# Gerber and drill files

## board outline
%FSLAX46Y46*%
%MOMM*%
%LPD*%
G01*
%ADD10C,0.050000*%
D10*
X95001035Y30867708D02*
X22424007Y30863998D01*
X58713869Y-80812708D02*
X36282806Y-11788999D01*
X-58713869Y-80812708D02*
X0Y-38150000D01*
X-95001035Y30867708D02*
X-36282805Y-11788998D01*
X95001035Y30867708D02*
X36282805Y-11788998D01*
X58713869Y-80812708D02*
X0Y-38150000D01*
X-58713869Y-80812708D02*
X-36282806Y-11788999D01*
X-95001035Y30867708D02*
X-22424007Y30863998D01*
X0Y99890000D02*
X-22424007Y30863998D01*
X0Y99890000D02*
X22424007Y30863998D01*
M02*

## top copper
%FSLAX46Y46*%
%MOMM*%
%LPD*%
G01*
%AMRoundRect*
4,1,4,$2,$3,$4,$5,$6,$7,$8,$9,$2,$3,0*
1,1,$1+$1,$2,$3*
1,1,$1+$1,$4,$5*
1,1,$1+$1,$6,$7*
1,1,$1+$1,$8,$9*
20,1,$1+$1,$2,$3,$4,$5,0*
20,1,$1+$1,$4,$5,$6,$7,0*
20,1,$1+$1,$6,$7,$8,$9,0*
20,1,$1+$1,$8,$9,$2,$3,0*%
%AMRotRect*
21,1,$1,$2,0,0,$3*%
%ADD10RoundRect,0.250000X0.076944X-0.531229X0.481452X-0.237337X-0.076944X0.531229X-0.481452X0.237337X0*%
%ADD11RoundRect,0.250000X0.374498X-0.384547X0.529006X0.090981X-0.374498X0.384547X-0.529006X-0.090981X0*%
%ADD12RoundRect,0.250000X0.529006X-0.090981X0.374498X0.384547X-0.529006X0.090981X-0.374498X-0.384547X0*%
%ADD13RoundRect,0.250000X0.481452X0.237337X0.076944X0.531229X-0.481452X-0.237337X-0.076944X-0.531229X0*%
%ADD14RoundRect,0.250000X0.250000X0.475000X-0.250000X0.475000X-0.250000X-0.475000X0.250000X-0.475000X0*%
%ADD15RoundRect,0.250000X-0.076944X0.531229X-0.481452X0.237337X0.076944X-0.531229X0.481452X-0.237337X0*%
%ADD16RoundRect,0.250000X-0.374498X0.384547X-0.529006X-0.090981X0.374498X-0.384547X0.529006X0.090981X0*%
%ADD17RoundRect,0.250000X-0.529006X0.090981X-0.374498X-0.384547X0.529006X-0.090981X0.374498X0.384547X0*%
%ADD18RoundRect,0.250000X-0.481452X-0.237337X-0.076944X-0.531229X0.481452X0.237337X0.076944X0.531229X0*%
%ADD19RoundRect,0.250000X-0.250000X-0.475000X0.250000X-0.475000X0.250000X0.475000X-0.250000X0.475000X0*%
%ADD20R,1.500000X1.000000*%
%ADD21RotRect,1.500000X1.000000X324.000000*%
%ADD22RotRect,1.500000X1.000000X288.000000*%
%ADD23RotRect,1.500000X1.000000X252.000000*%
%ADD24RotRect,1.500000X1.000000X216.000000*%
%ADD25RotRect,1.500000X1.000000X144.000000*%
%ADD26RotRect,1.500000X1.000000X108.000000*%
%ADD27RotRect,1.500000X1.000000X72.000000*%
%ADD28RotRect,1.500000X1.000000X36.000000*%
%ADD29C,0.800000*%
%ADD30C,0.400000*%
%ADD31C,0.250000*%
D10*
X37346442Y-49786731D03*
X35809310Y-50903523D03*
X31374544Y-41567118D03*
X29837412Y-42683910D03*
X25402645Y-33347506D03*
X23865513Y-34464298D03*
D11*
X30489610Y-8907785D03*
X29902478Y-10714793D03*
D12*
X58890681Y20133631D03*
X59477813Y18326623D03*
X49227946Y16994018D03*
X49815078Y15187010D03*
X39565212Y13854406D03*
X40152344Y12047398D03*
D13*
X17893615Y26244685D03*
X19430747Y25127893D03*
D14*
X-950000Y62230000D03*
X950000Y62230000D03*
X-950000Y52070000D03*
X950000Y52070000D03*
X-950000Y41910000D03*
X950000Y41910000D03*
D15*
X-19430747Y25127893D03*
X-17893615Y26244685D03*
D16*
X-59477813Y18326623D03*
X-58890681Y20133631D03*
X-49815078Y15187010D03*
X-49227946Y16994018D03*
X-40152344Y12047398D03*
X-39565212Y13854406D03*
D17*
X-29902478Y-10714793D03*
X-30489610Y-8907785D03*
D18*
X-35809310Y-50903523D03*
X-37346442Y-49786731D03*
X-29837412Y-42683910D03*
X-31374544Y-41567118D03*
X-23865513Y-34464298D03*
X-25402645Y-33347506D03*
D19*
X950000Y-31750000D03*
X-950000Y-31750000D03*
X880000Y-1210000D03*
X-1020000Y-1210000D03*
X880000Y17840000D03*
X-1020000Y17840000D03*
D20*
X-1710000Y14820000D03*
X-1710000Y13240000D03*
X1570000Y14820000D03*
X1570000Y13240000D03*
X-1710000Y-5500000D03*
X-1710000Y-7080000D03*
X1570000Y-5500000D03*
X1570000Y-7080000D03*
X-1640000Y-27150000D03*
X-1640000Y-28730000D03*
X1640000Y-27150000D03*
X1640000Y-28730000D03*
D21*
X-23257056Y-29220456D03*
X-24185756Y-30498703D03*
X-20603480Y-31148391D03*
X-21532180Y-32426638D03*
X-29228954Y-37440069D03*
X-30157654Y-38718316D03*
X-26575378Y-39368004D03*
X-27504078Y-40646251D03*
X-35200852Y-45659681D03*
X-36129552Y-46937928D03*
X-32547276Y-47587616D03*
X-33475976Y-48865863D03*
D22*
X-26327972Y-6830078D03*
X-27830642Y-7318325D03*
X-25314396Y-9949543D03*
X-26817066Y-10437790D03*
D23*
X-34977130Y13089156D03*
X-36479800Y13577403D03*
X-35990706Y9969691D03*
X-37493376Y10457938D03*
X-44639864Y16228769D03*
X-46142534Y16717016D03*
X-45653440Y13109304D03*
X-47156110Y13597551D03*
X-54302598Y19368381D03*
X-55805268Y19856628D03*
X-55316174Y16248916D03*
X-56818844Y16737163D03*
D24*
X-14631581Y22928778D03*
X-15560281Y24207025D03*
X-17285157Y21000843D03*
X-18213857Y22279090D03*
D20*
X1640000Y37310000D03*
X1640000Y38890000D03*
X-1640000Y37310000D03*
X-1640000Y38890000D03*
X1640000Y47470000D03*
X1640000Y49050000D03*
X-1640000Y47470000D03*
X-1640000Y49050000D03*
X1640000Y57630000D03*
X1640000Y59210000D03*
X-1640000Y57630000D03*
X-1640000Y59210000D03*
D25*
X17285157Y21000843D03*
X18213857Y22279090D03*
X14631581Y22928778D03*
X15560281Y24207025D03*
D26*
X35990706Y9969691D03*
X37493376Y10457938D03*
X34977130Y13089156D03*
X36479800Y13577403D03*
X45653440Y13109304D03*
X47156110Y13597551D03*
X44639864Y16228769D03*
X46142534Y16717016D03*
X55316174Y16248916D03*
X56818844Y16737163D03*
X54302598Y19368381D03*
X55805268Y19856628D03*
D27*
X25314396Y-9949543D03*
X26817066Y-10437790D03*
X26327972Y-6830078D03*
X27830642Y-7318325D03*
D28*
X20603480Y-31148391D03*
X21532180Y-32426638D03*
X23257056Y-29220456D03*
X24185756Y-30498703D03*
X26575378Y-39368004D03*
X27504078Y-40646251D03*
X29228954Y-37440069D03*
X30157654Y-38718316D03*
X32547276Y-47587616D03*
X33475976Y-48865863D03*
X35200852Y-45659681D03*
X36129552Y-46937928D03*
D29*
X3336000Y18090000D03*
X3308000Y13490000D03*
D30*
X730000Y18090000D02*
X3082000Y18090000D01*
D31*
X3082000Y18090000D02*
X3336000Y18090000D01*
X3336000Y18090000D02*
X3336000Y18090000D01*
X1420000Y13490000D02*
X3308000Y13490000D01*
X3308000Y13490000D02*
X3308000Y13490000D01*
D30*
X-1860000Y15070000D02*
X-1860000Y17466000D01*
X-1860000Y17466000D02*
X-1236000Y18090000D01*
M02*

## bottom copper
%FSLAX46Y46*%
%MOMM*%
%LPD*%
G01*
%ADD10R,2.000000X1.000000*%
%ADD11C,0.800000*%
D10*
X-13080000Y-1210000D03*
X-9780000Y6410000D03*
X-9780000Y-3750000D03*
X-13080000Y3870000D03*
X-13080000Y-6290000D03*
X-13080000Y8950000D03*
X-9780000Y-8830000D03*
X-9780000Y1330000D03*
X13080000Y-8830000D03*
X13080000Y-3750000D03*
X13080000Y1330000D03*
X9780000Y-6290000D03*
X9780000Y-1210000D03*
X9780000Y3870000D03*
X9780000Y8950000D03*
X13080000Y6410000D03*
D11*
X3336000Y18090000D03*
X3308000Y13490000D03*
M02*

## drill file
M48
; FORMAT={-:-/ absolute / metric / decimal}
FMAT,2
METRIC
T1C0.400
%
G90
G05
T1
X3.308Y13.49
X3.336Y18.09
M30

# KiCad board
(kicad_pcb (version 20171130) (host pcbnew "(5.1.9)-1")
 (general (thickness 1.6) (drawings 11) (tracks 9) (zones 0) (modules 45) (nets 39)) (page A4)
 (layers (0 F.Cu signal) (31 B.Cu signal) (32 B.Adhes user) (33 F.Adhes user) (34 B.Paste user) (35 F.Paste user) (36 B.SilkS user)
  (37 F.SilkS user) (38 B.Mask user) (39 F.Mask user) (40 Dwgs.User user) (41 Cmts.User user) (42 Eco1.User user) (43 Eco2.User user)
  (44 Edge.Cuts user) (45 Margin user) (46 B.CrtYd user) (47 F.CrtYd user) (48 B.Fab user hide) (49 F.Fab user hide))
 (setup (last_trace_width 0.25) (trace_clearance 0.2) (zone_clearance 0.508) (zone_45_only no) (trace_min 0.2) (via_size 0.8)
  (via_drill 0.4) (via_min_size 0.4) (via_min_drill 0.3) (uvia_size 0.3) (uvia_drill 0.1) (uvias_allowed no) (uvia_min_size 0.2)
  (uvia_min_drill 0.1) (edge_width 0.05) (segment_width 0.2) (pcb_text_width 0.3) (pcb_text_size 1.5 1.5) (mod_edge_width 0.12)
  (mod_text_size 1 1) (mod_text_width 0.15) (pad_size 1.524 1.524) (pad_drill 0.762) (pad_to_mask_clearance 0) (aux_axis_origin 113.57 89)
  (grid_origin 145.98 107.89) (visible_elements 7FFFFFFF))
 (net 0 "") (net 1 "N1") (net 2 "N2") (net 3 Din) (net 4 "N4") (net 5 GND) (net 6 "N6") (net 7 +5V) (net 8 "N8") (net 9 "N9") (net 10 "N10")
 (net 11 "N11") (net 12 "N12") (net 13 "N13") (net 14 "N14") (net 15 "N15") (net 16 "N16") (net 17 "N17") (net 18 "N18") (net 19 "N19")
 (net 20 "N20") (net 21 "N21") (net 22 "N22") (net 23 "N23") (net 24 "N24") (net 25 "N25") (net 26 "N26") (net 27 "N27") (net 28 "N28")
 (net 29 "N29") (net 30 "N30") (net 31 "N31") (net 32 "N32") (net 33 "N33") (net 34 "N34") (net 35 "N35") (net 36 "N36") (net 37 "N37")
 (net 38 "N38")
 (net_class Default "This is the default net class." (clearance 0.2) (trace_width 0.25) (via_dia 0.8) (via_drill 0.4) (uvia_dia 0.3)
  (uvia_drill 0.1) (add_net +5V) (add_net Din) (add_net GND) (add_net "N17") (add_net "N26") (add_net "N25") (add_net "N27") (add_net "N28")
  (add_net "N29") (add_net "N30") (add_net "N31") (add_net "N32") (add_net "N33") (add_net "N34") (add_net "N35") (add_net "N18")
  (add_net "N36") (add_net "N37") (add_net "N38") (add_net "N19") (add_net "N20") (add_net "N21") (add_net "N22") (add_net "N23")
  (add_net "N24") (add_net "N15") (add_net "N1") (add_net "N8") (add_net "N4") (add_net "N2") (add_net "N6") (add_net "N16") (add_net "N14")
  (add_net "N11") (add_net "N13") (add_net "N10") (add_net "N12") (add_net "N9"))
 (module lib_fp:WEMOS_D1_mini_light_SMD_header (layer B.Cu) (at 0 -0.06 180)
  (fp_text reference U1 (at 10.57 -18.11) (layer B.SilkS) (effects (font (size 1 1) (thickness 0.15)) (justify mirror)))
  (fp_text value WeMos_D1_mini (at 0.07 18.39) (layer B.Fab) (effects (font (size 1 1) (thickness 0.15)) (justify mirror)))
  (pad 12 smd rect (at 13.08 -1.27 180) (size 2 1) (layers B.Cu B.Paste B.Mask) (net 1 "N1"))
  (pad 15 smd rect (at 9.78 6.35 180) (size 2 1) (layers B.Cu B.Paste B.Mask) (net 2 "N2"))
  (pad 11 smd rect (at 9.78 -3.81 180) (size 2 1) (layers B.Cu B.Paste B.Mask) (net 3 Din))
  (pad 14 smd rect (at 13.08 3.81 180) (size 2 1) (layers B.Cu B.Paste B.Mask) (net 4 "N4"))
  (pad 10 smd rect (at 13.08 -6.35 180) (size 2 1) (layers B.Cu B.Paste B.Mask) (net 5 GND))
  (pad 16 smd rect (at 13.08 8.89 180) (size 2 1) (layers B.Cu B.Paste B.Mask) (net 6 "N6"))
  (pad 9 smd rect (at 9.78 -8.89 180) (size 2 1) (layers B.Cu B.Paste B.Mask) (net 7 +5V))
  (pad 13 smd rect (at 9.78 1.27 180) (size 2 1) (layers B.Cu B.Paste B.Mask) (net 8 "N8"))
  (pad 8 smd rect (at -13.08 -8.89 180) (size 2 1) (layers B.Cu B.Paste B.Mask) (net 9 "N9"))
  (pad 6 smd rect (at -13.08 -3.81 180) (size 2 1) (layers B.Cu B.Paste B.Mask) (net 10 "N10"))
  (pad 4 smd rect (at -13.08 1.27 180) (size 2 1) (layers B.Cu B.Paste B.Mask) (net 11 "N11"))
  (pad 7 smd rect (at -9.78 -6.35 180) (size 2 1) (layers B.Cu B.Paste B.Mask) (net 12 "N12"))
  (pad 5 smd rect (at -9.78 -1.27 180) (size 2 1) (layers B.Cu B.Paste B.Mask) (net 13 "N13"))
  (pad 3 smd rect (at -9.78 3.81 180) (size 2 1) (layers B.Cu B.Paste B.Mask) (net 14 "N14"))
  (pad 1 smd rect (at -9.78 8.89 180) (size 2 1) (layers B.Cu B.Paste B.Mask) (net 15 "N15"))
  (pad 2 smd rect (at -13.08 6.35 180) (size 2 1) (layers B.Cu B.Paste B.Mask) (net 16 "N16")))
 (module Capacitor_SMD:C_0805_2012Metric (layer F.Cu) (at 36.577876 50.345127 36)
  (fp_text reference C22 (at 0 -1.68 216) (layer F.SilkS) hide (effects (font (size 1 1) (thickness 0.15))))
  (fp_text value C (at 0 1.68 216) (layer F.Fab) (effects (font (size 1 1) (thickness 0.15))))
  (pad 2 smd roundrect (at 0.95 0 36) (size 1 1.45) (layers F.Cu F.Paste F.Mask) (roundrect_rratio 0.25) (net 5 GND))
  (pad 1 smd roundrect (at -0.95 0 36) (size 1 1.45) (layers F.Cu F.Paste F.Mask) (roundrect_rratio 0.25) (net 7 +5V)))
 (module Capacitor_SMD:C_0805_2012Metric (layer F.Cu) (at 30.605978 42.125514 36)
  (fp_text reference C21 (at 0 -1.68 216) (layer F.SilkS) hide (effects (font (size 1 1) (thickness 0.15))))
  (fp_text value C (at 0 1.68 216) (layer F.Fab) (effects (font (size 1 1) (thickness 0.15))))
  (pad 2 smd roundrect (at 0.95 0 36) (size 1 1.45) (layers F.Cu F.Paste F.Mask) (roundrect_rratio 0.25) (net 5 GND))
  (pad 1 smd roundrect (at -0.95 0 36) (size 1 1.45) (layers F.Cu F.Paste F.Mask) (roundrect_rratio 0.25) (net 7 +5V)))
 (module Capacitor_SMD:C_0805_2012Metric (layer F.Cu) (at 24.634079 33.905902 36)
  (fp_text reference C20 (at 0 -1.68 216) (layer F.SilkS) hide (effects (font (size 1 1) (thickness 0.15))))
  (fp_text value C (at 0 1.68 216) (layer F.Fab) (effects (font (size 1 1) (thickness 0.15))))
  (pad 2 smd roundrect (at 0.95 0 36) (size 1 1.45) (layers F.Cu F.Paste F.Mask) (roundrect_rratio 0.25) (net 5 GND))
  (pad 1 smd roundrect (at -0.95 0 36) (size 1 1.45) (layers F.Cu F.Paste F.Mask) (roundrect_rratio 0.25) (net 7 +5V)))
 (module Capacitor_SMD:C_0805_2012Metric (layer F.Cu) (at 30.196044 9.811289 72)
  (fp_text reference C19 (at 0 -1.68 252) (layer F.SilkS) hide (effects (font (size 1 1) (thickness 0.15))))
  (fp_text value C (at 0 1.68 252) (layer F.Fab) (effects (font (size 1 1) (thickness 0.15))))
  (pad 2 smd roundrect (at 0.95 0 72) (size 1 1.45) (layers F.Cu F.Paste F.Mask) (roundrect_rratio 0.25) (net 5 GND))
  (pad 1 smd roundrect (at -0.95 0 72) (size 1 1.45) (layers F.Cu F.Paste F.Mask) (roundrect_rratio 0.25) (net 7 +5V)))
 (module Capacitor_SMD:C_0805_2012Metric (layer F.Cu) (at 59.184247 -19.230127 108)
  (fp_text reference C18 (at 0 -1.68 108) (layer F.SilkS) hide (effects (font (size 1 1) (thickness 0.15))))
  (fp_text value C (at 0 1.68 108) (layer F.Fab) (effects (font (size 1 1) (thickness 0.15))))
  (pad 2 smd roundrect (at 0.95 0 108) (size 1 1.45) (layers F.Cu F.Paste F.Mask) (roundrect_rratio 0.25) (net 5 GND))
  (pad 1 smd roundrect (at -0.95 0 108) (size 1 1.45) (layers F.Cu F.Paste F.Mask) (roundrect_rratio 0.25) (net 7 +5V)))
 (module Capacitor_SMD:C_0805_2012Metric (layer F.Cu) (at 49.521512 -16.090514 108)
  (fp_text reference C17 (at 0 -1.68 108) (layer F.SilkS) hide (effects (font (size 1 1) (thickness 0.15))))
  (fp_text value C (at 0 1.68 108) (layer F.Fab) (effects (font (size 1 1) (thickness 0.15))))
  (pad 2 smd roundrect (at 0.95 0 108) (size 1 1.45) (layers F.Cu F.Paste F.Mask) (roundrect_rratio 0.25) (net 5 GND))
  (pad 1 smd roundrect (at -0.95 0 108) (size 1 1.45) (layers F.Cu F.Paste F.Mask) (roundrect_rratio 0.25) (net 7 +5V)))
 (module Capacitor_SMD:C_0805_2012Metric (layer F.Cu) (at 39.858778 -12.950902 108)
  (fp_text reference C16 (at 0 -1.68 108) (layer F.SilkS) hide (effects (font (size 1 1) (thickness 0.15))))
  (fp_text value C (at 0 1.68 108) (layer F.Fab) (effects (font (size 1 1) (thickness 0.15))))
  (pad 2 smd roundrect (at 0.95 0 108) (size 1 1.45) (layers F.Cu F.Paste F.Mask) (roundrect_rratio 0.25) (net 5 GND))
  (pad 1 smd roundrect (at -0.95 0 108) (size 1 1.45) (layers F.Cu F.Paste F.Mask) (roundrect_rratio 0.25) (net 7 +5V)))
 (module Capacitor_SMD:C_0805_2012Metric (layer F.Cu) (at 18.662181 -25.686289 144)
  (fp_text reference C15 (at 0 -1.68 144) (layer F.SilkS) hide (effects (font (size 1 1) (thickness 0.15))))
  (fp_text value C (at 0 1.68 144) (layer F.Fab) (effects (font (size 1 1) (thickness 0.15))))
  (pad 2 smd roundrect (at 0.95 0 144) (size 1 1.45) (layers F.Cu F.Paste F.Mask) (roundrect_rratio 0.25) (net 5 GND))
  (pad 1 smd roundrect (at -0.95 0 144) (size 1 1.45) (layers F.Cu F.Paste F.Mask) (roundrect_rratio 0.25) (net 7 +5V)))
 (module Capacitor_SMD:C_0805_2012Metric (layer F.Cu) (at 0 -62.23 180)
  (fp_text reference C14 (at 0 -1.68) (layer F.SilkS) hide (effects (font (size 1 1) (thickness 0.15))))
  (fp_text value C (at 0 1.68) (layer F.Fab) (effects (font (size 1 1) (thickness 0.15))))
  (pad 2 smd roundrect (at 0.95 0 180) (size 1 1.45) (layers F.Cu F.Paste F.Mask) (roundrect_rratio 0.25) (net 5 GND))
  (pad 1 smd roundrect (at -0.95 0 180) (size 1 1.45) (layers F.Cu F.Paste F.Mask) (roundrect_rratio 0.25) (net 7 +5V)))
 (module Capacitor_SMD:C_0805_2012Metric (layer F.Cu) (at 0 -52.07 180)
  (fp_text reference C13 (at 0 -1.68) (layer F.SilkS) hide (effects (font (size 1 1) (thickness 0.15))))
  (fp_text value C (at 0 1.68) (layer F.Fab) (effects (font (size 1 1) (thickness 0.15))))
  (pad 2 smd roundrect (at 0.95 0 180) (size 1 1.45) (layers F.Cu F.Paste F.Mask) (roundrect_rratio 0.25) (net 5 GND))
  (pad 1 smd roundrect (at -0.95 0 180) (size 1 1.45) (layers F.Cu F.Paste F.Mask) (roundrect_rratio 0.25) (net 7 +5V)))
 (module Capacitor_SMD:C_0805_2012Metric (layer F.Cu) (at 0 -41.91 180)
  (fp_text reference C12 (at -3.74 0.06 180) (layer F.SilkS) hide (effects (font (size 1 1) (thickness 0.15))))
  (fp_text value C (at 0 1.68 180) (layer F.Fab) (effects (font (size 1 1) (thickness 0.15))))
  (pad 2 smd roundrect (at 0.95 0 180) (size 1 1.45) (layers F.Cu F.Paste F.Mask) (roundrect_rratio 0.25) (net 5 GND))
  (pad 1 smd roundrect (at -0.95 0 180) (size 1 1.45) (layers F.Cu F.Paste F.Mask) (roundrect_rratio 0.25) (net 7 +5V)))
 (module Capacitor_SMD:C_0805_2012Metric (layer F.Cu) (at -18.662181 -25.686289 216)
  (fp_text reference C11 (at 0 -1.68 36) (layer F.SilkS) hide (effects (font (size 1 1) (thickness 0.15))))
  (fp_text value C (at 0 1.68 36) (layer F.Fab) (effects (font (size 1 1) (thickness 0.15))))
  (pad 2 smd roundrect (at 0.95 0 216) (size 1 1.45) (layers F.Cu F.Paste F.Mask) (roundrect_rratio 0.25) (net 5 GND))
  (pad 1 smd roundrect (at -0.95 0 216) (size 1 1.45) (layers F.Cu F.Paste F.Mask) (roundrect_rratio 0.25) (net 7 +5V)))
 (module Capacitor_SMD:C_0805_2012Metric (layer F.Cu) (at -59.184247 -19.230127 252)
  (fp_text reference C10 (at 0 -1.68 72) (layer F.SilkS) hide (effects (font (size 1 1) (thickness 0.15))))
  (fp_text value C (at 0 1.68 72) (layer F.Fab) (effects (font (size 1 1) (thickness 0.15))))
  (pad 2 smd roundrect (at 0.95 0 252) (size 1 1.45) (layers F.Cu F.Paste F.Mask) (roundrect_rratio 0.25) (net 5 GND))
  (pad 1 smd roundrect (at -0.95 0 252) (size 1 1.45) (layers F.Cu F.Paste F.Mask) (roundrect_rratio 0.25) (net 7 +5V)))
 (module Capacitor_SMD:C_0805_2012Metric (layer F.Cu) (at -49.521512 -16.090514 252)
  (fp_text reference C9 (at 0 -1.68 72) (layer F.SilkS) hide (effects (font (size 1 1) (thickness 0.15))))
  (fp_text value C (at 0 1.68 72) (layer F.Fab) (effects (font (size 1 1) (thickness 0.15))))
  (pad 2 smd roundrect (at 0.95 0 252) (size 1 1.45) (layers F.Cu F.Paste F.Mask) (roundrect_rratio 0.25) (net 5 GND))
  (pad 1 smd roundrect (at -0.95 0 252) (size 1 1.45) (layers F.Cu F.Paste F.Mask) (roundrect_rratio 0.25) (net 7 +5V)))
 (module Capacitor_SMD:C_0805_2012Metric (layer F.Cu) (at -39.858778 -12.950902 252)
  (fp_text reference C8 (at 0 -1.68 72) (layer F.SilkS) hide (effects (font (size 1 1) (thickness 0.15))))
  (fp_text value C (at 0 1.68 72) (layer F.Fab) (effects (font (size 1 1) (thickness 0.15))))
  (pad 2 smd roundrect (at 0.95 0 252) (size 1 1.45) (layers F.Cu F.Paste F.Mask) (roundrect_rratio 0.25) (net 5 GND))
  (pad 1 smd roundrect (at -0.95 0 252) (size 1 1.45) (layers F.Cu F.Paste F.Mask) (roundrect_rratio 0.25) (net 7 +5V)))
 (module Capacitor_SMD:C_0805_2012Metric (layer F.Cu) (at -30.196044 9.811289 288)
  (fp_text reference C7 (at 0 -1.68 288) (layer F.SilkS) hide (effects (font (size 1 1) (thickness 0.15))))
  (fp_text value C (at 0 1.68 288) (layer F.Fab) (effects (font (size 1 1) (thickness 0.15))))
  (pad 2 smd roundrect (at 0.95 0 288) (size 1 1.45) (layers F.Cu F.Paste F.Mask) (roundrect_rratio 0.25) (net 5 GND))
  (pad 1 smd roundrect (at -0.95 0 288) (size 1 1.45) (layers F.Cu F.Paste F.Mask) (roundrect_rratio 0.25) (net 7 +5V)))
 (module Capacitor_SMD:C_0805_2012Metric (layer F.Cu) (at -36.577876 50.345127 324)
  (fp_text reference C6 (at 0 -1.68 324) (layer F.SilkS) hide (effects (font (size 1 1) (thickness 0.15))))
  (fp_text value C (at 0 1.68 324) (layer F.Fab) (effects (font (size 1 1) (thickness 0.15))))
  (pad 2 smd roundrect (at 0.95 0 324) (size 1 1.45) (layers F.Cu F.Paste F.Mask) (roundrect_rratio 0.25) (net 5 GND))
  (pad 1 smd roundrect (at -0.95 0 324) (size 1 1.45) (layers F.Cu F.Paste F.Mask) (roundrect_rratio 0.25) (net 7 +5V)))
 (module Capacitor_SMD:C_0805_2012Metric (layer F.Cu) (at -30.605978 42.125514 324)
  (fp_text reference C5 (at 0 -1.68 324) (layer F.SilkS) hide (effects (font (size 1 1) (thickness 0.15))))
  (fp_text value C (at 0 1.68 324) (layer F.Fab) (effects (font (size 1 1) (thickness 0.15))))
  (pad 2 smd roundrect (at 0.95 0 324) (size 1 1.45) (layers F.Cu F.Paste F.Mask) (roundrect_rratio 0.25) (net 5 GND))
  (pad 1 smd roundrect (at -0.95 0 324) (size 1 1.45) (layers F.Cu F.Paste F.Mask) (roundrect_rratio 0.25) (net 7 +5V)))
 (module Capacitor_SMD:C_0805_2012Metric (layer F.Cu) (at -24.634079 33.905902 324)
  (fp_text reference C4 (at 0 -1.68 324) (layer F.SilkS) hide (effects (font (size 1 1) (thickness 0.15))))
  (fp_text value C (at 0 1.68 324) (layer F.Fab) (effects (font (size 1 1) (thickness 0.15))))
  (pad 2 smd roundrect (at 0.95 0 324) (size 1 1.45) (layers F.Cu F.Paste F.Mask) (roundrect_rratio 0.25) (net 5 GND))
  (pad 1 smd roundrect (at -0.95 0 324) (size 1 1.45) (layers F.Cu F.Paste F.Mask) (roundrect_rratio 0.25) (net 7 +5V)))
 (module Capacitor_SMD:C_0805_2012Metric (layer F.Cu) (at 0 31.75)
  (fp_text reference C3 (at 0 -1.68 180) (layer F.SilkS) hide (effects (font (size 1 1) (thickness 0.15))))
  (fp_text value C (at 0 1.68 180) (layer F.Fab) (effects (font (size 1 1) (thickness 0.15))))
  (pad 2 smd roundrect (at 0.95 0) (size 1 1.45) (layers F.Cu F.Paste F.Mask) (roundrect_rratio 0.25) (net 5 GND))
  (pad 1 smd roundrect (at -0.95 0) (size 1 1.45) (layers F.Cu F.Paste F.Mask) (roundrect_rratio 0.25) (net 7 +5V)))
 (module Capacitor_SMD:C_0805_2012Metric (layer F.Cu) (at -0.07 1.21)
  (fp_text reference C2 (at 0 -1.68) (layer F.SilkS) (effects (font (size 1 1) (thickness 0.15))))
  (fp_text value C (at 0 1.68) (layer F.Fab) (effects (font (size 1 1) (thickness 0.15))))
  (pad 2 smd roundrect (at 0.95 0) (size 1 1.45) (layers F.Cu F.Paste F.Mask) (roundrect_rratio 0.25) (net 5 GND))
  (pad 1 smd roundrect (at -0.95 0) (size 1 1.45) (layers F.Cu F.Paste F.Mask) (roundrect_rratio 0.25) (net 7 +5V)))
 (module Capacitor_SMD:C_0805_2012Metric (layer F.Cu) (at -0.07 -17.84)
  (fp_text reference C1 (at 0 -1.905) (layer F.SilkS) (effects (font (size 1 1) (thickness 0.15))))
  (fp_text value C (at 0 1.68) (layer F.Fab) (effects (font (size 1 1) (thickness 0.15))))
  (pad 2 smd roundrect (at 0.95 0) (size 1 1.45) (layers F.Cu F.Paste F.Mask) (roundrect_rratio 0.25) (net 5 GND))
  (pad 1 smd roundrect (at -0.95 0) (size 1 1.45) (layers F.Cu F.Paste F.Mask) (roundrect_rratio 0.25) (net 7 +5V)))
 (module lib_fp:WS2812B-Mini (layer F.Cu) (at -0.07 -14.03)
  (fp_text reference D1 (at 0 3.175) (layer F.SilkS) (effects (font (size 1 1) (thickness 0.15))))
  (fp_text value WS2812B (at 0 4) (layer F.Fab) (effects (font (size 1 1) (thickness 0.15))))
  (pad 1 smd rect (at -1.64 -0.79) (size 1.5 1) (layers F.Cu F.Paste F.Mask) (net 7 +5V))
  (pad 2 smd rect (at -1.64 0.79) (size 1.5 1) (layers F.Cu F.Paste F.Mask) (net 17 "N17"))
  (pad 4 smd rect (at 1.64 -0.79) (size 1.5 1) (layers F.Cu F.Paste F.Mask) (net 3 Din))
  (pad 3 smd rect (at 1.64 0.79) (size 1.5 1) (layers F.Cu F.Paste F.Mask) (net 5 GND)))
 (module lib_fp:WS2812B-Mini (layer F.Cu) (at -0.07 6.29)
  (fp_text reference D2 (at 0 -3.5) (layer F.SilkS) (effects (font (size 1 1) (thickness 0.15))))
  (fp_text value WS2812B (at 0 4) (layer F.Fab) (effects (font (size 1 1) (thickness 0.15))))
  (pad 1 smd rect (at -1.64 -0.79) (size 1.5 1) (layers F.Cu F.Paste F.Mask) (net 7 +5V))
  (pad 2 smd rect (at -1.64 0.79) (size 1.5 1) (layers F.Cu F.Paste F.Mask) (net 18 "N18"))
  (pad 4 smd rect (at 1.64 -0.79) (size 1.5 1) (layers F.Cu F.Paste F.Mask) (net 17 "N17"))
  (pad 3 smd rect (at 1.64 0.79) (size 1.5 1) (layers F.Cu F.Paste F.Mask) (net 5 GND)))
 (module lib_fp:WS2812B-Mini (layer F.Cu) (at 0 27.94)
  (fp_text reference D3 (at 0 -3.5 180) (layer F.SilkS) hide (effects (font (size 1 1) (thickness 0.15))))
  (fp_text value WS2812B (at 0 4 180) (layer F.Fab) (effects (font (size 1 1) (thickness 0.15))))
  (pad 1 smd rect (at -1.64 -0.79) (size 1.5 1) (layers F.Cu F.Paste F.Mask) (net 7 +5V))
  (pad 2 smd rect (at -1.64 0.79) (size 1.5 1) (layers F.Cu F.Paste F.Mask) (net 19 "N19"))
  (pad 4 smd rect (at 1.64 -0.79) (size 1.5 1) (layers F.Cu F.Paste F.Mask) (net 18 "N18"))
  (pad 3 smd rect (at 1.64 0.79) (size 1.5 1) (layers F.Cu F.Paste F.Mask) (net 5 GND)))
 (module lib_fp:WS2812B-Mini (layer F.Cu) (at -22.394618 30.823547 324)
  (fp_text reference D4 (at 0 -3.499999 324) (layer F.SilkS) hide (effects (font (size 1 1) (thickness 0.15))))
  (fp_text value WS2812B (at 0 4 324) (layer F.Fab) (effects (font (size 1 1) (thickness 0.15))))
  (pad 1 smd rect (at -1.64 -0.79 324) (size 1.5 1) (layers F.Cu F.Paste F.Mask) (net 7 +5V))
  (pad 2 smd rect (at -1.64 0.79 324) (size 1.5 1) (layers F.Cu F.Paste F.Mask) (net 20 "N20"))
  (pad 4 smd rect (at 1.64 -0.79 324) (size 1.5 1) (layers F.Cu F.Paste F.Mask) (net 19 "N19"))
  (pad 3 smd rect (at 1.64 0.79 324) (size 1.5 1) (layers F.Cu F.Paste F.Mask) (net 5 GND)))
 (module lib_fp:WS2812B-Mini (layer F.Cu) (at -28.366516 39.04316 324)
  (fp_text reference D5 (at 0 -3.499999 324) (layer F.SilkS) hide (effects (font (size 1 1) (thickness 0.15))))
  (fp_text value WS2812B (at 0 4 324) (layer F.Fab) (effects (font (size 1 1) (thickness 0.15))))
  (pad 1 smd rect (at -1.64 -0.79 324) (size 1.5 1) (layers F.Cu F.Paste F.Mask) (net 7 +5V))
  (pad 2 smd rect (at -1.64 0.79 324) (size 1.5 1) (layers F.Cu F.Paste F.Mask) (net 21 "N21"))
  (pad 4 smd rect (at 1.64 -0.79 324) (size 1.5 1) (layers F.Cu F.Paste F.Mask) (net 20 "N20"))
  (pad 3 smd rect (at 1.64 0.79 324) (size 1.5 1) (layers F.Cu F.Paste F.Mask) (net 5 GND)))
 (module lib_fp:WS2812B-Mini (layer F.Cu) (at -34.338414 47.262772 324)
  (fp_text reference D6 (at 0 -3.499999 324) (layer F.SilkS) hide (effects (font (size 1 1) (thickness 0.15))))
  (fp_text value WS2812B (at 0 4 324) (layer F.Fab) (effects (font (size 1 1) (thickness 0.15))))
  (pad 1 smd rect (at -1.64 -0.79 324) (size 1.5 1) (layers F.Cu F.Paste F.Mask) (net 7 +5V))
  (pad 2 smd rect (at -1.64 0.79 324) (size 1.5 1) (layers F.Cu F.Paste F.Mask) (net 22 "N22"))
  (pad 4 smd rect (at 1.64 -0.79 324) (size 1.5 1) (layers F.Cu F.Paste F.Mask) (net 21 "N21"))
  (pad 3 smd rect (at 1.64 0.79 324) (size 1.5 1) (layers F.Cu F.Paste F.Mask) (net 5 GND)))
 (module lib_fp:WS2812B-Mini (layer F.Cu) (at -26.572519 8.633934 288)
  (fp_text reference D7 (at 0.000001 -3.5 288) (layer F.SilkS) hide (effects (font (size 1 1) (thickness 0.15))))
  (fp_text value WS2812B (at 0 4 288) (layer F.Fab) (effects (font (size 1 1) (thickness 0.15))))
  (pad 1 smd rect (at -1.64 -0.79 288) (size 1.5 1) (layers F.Cu F.Paste F.Mask) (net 7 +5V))
  (pad 2 smd rect (at -1.64 0.79 288) (size 1.5 1) (layers F.Cu F.Paste F.Mask) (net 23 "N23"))
  (pad 4 smd rect (at 1.64 -0.79 288) (size 1.5 1) (layers F.Cu F.Paste F.Mask) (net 22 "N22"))
  (pad 3 smd rect (at 1.64 0.79 288) (size 1.5 1) (layers F.Cu F.Paste F.Mask) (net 5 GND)))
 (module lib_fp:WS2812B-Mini (layer F.Cu) (at -36.235253 -11.773547 252)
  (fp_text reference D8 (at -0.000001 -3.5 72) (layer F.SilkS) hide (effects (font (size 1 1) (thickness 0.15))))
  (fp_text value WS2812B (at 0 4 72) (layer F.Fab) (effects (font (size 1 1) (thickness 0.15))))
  (pad 1 smd rect (at -1.64 -0.79 252) (size 1.5 1) (layers F.Cu F.Paste F.Mask) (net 7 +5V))
  (pad 2 smd rect (at -1.64 0.79 252) (size 1.5 1) (layers F.Cu F.Paste F.Mask) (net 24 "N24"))
  (pad 4 smd rect (at 1.64 -0.79 252) (size 1.5 1) (layers F.Cu F.Paste F.Mask) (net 23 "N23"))
  (pad 3 smd rect (at 1.64 0.79 252) (size 1.5 1) (layers F.Cu F.Paste F.Mask) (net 5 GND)))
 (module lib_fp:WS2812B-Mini (layer F.Cu) (at -45.897987 -14.91316 252)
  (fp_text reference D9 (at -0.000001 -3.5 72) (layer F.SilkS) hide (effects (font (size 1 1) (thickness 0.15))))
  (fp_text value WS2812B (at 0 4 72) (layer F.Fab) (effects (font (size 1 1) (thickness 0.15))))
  (pad 1 smd rect (at -1.64 -0.79 252) (size 1.5 1) (layers F.Cu F.Paste F.Mask) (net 7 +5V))
  (pad 2 smd rect (at -1.64 0.79 252) (size 1.5 1) (layers F.Cu F.Paste F.Mask) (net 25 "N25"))
  (pad 4 smd rect (at 1.64 -0.79 252) (size 1.5 1) (layers F.Cu F.Paste F.Mask) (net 24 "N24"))
  (pad 3 smd rect (at 1.64 0.79 252) (size 1.5 1) (layers F.Cu F.Paste F.Mask) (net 5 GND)))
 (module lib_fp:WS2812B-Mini (layer F.Cu) (at -55.560721 -18.052772 252)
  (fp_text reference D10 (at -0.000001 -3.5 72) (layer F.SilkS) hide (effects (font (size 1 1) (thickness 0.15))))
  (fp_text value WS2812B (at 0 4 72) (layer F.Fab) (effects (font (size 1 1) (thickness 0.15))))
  (pad 1 smd rect (at -1.64 -0.79 252) (size 1.5 1) (layers F.Cu F.Paste F.Mask) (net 7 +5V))
  (pad 2 smd rect (at -1.64 0.79 252) (size 1.5 1) (layers F.Cu F.Paste F.Mask) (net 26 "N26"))
  (pad 4 smd rect (at 1.64 -0.79 252) (size 1.5 1) (layers F.Cu F.Paste F.Mask) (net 25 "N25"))
  (pad 3 smd rect (at 1.64 0.79 252) (size 1.5 1) (layers F.Cu F.Paste F.Mask) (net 5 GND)))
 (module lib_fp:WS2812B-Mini (layer F.Cu) (at -16.422719 -22.603934 216)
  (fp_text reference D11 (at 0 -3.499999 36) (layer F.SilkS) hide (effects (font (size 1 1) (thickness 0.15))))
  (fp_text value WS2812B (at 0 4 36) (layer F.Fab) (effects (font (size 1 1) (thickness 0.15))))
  (pad 1 smd rect (at -1.64 -0.79 216) (size 1.5 1) (layers F.Cu F.Paste F.Mask) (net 7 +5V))
  (pad 2 smd rect (at -1.64 0.79 216) (size 1.5 1) (layers F.Cu F.Paste F.Mask) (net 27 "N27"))
  (pad 4 smd rect (at 1.64 -0.79 216) (size 1.5 1) (layers F.Cu F.Paste F.Mask) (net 26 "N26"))
  (pad 3 smd rect (at 1.64 0.79 216) (size 1.5 1) (layers F.Cu F.Paste F.Mask) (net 5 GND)))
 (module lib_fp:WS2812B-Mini (layer F.Cu) (at 0 -38.1 180)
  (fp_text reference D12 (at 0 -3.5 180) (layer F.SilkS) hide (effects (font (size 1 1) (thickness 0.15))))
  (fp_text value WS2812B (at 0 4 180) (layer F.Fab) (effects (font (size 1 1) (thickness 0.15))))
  (pad 1 smd rect (at -1.64 -0.79 180) (size 1.5 1) (layers F.Cu F.Paste F.Mask) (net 7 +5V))
  (pad 2 smd rect (at -1.64 0.79 180) (size 1.5 1) (layers F.Cu F.Paste F.Mask) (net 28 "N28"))
  (pad 4 smd rect (at 1.64 -0.79 180) (size 1.5 1) (layers F.Cu F.Paste F.Mask) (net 27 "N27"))
  (pad 3 smd rect (at 1.64 0.79 180) (size 1.5 1) (layers F.Cu F.Paste F.Mask) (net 5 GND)))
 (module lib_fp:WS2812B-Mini (layer F.Cu) (at 0 -48.26 180)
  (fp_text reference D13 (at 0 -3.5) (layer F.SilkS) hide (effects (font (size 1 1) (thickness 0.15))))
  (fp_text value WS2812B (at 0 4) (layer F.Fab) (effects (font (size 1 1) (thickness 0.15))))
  (pad 1 smd rect (at -1.64 -0.79 180) (size 1.5 1) (layers F.Cu F.Paste F.Mask) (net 7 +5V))
  (pad 2 smd rect (at -1.64 0.79 180) (size 1.5 1) (layers F.Cu F.Paste F.Mask) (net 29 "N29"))
  (pad 4 smd rect (at 1.64 -0.79 180) (size 1.5 1) (layers F.Cu F.Paste F.Mask) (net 28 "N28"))
  (pad 3 smd rect (at 1.64 0.79 180) (size 1.5 1) (layers F.Cu F.Paste F.Mask) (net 5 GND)))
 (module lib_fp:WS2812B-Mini (layer F.Cu) (at 0 -58.42 180)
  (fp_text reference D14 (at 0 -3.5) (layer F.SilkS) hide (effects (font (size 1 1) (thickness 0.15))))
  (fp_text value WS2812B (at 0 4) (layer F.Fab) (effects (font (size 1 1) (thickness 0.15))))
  (pad 1 smd rect (at -1.64 -0.79 180) (size 1.5 1) (layers F.Cu F.Paste F.Mask) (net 7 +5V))
  (pad 2 smd rect (at -1.64 0.79 180) (size 1.5 1) (layers F.Cu F.Paste F.Mask) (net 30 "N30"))
  (pad 4 smd rect (at 1.64 -0.79 180) (size 1.5 1) (layers F.Cu F.Paste F.Mask) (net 29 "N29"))
  (pad 3 smd rect (at 1.64 0.79 180) (size 1.5 1) (layers F.Cu F.Paste F.Mask) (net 5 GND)))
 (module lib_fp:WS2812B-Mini (layer F.Cu) (at 16.422719 -22.603934 144)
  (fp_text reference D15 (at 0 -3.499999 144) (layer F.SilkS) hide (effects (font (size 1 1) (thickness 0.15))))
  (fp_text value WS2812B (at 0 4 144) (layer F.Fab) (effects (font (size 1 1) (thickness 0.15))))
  (pad 1 smd rect (at -1.64 -0.79 144) (size 1.5 1) (layers F.Cu F.Paste F.Mask) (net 7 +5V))
  (pad 2 smd rect (at -1.64 0.79 144) (size 1.5 1) (layers F.Cu F.Paste F.Mask) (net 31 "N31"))
  (pad 4 smd rect (at 1.64 -0.79 144) (size 1.5 1) (layers F.Cu F.Paste F.Mask) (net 30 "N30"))
  (pad 3 smd rect (at 1.64 0.79 144) (size 1.5 1) (layers F.Cu F.Paste F.Mask) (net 5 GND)))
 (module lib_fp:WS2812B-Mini (layer F.Cu) (at 36.235253 -11.773547 108)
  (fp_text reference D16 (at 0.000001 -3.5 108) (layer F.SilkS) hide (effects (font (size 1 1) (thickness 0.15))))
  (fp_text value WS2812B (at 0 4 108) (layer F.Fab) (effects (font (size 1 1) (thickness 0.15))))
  (pad 1 smd rect (at -1.64 -0.79 108) (size 1.5 1) (layers F.Cu F.Paste F.Mask) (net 7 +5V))
  (pad 2 smd rect (at -1.64 0.79 108) (size 1.5 1) (layers F.Cu F.Paste F.Mask) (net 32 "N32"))
  (pad 4 smd rect (at 1.64 -0.79 108) (size 1.5 1) (layers F.Cu F.Paste F.Mask) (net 31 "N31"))
  (pad 3 smd rect (at 1.64 0.79 108) (size 1.5 1) (layers F.Cu F.Paste F.Mask) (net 5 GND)))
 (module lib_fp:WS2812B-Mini (layer F.Cu) (at 45.897987 -14.91316 108)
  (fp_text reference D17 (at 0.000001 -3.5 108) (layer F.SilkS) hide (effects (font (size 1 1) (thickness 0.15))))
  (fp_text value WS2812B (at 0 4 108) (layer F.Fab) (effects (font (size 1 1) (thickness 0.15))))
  (pad 1 smd rect (at -1.64 -0.79 108) (size 1.5 1) (layers F.Cu F.Paste F.Mask) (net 7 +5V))
  (pad 2 smd rect (at -1.64 0.79 108) (size 1.5 1) (layers F.Cu F.Paste F.Mask) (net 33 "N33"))
  (pad 4 smd rect (at 1.64 -0.79 108) (size 1.5 1) (layers F.Cu F.Paste F.Mask) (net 32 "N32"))
  (pad 3 smd rect (at 1.64 0.79 108) (size 1.5 1) (layers F.Cu F.Paste F.Mask) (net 5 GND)))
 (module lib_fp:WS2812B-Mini (layer F.Cu) (at 55.560721 -18.052772 108)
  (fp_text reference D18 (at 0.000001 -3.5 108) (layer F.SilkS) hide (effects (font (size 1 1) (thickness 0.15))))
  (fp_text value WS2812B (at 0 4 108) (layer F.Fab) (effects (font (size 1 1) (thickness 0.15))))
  (pad 1 smd rect (at -1.64 -0.79 108) (size 1.5 1) (layers F.Cu F.Paste F.Mask) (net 7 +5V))
  (pad 2 smd rect (at -1.64 0.79 108) (size 1.5 1) (layers F.Cu F.Paste F.Mask) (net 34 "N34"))
  (pad 4 smd rect (at 1.64 -0.79 108) (size 1.5 1) (layers F.Cu F.Paste F.Mask) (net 33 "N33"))
  (pad 3 smd rect (at 1.64 0.79 108) (size 1.5 1) (layers F.Cu F.Paste F.Mask) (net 5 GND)))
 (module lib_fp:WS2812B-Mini (layer F.Cu) (at 26.572519 8.633934 72)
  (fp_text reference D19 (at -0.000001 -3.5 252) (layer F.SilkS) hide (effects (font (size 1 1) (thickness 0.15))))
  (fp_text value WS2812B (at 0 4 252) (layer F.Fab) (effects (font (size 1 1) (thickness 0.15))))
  (pad 1 smd rect (at -1.64 -0.79 72) (size 1.5 1) (layers F.Cu F.Paste F.Mask) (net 7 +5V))
  (pad 2 smd rect (at -1.64 0.79 72) (size 1.5 1) (layers F.Cu F.Paste F.Mask) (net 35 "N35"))
  (pad 4 smd rect (at 1.64 -0.79 72) (size 1.5 1) (layers F.Cu F.Paste F.Mask) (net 34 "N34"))
  (pad 3 smd rect (at 1.64 0.79 72) (size 1.5 1) (layers F.Cu F.Paste F.Mask) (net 5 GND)))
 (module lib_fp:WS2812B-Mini (layer F.Cu) (at 22.394618 30.823547 36)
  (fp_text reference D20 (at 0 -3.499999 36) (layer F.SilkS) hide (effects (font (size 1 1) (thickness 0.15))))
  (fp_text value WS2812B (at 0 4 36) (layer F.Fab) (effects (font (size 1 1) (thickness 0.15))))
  (pad 1 smd rect (at -1.64 -0.79 36) (size 1.5 1) (layers F.Cu F.Paste F.Mask) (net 7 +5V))
  (pad 2 smd rect (at -1.64 0.79 36) (size 1.5 1) (layers F.Cu F.Paste F.Mask) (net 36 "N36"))
  (pad 4 smd rect (at 1.64 -0.79 36) (size 1.5 1) (layers F.Cu F.Paste F.Mask) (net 35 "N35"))
  (pad 3 smd rect (at 1.64 0.79 36) (size 1.5 1) (layers F.Cu F.Paste F.Mask) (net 5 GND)))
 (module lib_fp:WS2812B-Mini (layer F.Cu) (at 28.366516 39.04316 36)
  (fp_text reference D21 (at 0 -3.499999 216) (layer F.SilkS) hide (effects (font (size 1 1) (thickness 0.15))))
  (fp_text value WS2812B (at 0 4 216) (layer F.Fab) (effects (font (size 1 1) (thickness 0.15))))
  (pad 1 smd rect (at -1.64 -0.79 36) (size 1.5 1) (layers F.Cu F.Paste F.Mask) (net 7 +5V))
  (pad 2 smd rect (at -1.64 0.79 36) (size 1.5 1) (layers F.Cu F.Paste F.Mask) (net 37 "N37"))
  (pad 4 smd rect (at 1.64 -0.79 36) (size 1.5 1) (layers F.Cu F.Paste F.Mask) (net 36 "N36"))
  (pad 3 smd rect (at 1.64 0.79 36) (size 1.5 1) (layers F.Cu F.Paste F.Mask) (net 5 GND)))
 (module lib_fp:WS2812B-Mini (layer F.Cu) (at 34.338414 47.262772 36)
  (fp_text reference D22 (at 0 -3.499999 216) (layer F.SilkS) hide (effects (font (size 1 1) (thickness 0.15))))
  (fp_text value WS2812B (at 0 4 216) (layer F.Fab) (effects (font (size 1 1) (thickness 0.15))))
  (pad 1 smd rect (at -1.64 -0.79 36) (size 1.5 1) (layers F.Cu F.Paste F.Mask) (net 7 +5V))
  (pad 2 smd rect (at -1.64 0.79 36) (size 1.5 1) (layers F.Cu F.Paste F.Mask) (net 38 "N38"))
  (pad 4 smd rect (at 1.64 -0.79 36) (size 1.5 1) (layers F.Cu F.Paste F.Mask) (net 37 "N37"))
  (pad 3 smd rect (at 1.64 0.79 36) (size 1.5 1) (layers F.Cu F.Paste F.Mask) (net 5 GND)))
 (gr_line (start 95.001035 -30.867708) (end 22.424007 -30.863998) (layer Edge.Cuts) (width 0.05))
 (gr_line (start 58.713869 80.812708) (end 36.282806 11.788999) (layer Edge.Cuts) (width 0.05))
 (gr_line (start -58.713869 80.812708) (end 0 38.15) (layer Edge.Cuts) (width 0.05))
 (gr_line (start -95.001035 -30.867708) (end -36.282805 11.788998) (layer Edge.Cuts) (width 0.05))
 (gr_line (start 95.001035 -30.867708) (end 36.282805 11.788998) (layer Edge.Cuts) (width 0.05))
 (gr_line (start 58.713869 80.812708) (end 0 38.15) (layer Edge.Cuts) (width 0.05))
 (gr_line (start -58.713869 80.812708) (end -36.282806 11.788999) (layer Edge.Cuts) (width 0.05))
 (gr_line (start -95.001035 -30.867708) (end -22.424007 -30.863998) (layer Edge.Cuts) (width 0.05))
 (gr_line (start 0 -99.89) (end -22.424007 -30.863998) (layer Edge.Cuts) (width 0.05))
 (gr_line (start 0 -99.89) (end 22.424007 -30.863998) (layer Edge.Cuts) (width 0.05))
 (segment (start 0.73 -18.09) (end 3.082 -18.09) (width 0.4) (layer F.Cu) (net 5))
 (segment (start 3.082 -18.09) (end 3.336 -18.09) (width 0.25) (layer F.Cu) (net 5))
 (segment (start 3.336 -18.09) (end 3.336 -18.09) (width 0.25) (layer F.Cu) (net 5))
 (via (at 3.336 -18.09) (size 0.8) (drill 0.4) (layers F.Cu B.Cu) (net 5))
 (segment (start 1.42 -13.49) (end 3.308 -13.49) (width 0.25) (layer F.Cu) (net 5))
 (segment (start 3.308 -13.49) (end 3.308 -13.49) (width 0.25) (layer F.Cu) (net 5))
 (via (at 3.308 -13.49) (size 0.8) (drill 0.4) (layers F.Cu B.Cu) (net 5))
 (segment (start -1.86 -15.07) (end -1.86 -17.466) (width 0.4) (layer F.Cu) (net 7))
 (segment (start -1.86 -17.466) (end -1.236 -18.09) (width 0.4) (layer F.Cu) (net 7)))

